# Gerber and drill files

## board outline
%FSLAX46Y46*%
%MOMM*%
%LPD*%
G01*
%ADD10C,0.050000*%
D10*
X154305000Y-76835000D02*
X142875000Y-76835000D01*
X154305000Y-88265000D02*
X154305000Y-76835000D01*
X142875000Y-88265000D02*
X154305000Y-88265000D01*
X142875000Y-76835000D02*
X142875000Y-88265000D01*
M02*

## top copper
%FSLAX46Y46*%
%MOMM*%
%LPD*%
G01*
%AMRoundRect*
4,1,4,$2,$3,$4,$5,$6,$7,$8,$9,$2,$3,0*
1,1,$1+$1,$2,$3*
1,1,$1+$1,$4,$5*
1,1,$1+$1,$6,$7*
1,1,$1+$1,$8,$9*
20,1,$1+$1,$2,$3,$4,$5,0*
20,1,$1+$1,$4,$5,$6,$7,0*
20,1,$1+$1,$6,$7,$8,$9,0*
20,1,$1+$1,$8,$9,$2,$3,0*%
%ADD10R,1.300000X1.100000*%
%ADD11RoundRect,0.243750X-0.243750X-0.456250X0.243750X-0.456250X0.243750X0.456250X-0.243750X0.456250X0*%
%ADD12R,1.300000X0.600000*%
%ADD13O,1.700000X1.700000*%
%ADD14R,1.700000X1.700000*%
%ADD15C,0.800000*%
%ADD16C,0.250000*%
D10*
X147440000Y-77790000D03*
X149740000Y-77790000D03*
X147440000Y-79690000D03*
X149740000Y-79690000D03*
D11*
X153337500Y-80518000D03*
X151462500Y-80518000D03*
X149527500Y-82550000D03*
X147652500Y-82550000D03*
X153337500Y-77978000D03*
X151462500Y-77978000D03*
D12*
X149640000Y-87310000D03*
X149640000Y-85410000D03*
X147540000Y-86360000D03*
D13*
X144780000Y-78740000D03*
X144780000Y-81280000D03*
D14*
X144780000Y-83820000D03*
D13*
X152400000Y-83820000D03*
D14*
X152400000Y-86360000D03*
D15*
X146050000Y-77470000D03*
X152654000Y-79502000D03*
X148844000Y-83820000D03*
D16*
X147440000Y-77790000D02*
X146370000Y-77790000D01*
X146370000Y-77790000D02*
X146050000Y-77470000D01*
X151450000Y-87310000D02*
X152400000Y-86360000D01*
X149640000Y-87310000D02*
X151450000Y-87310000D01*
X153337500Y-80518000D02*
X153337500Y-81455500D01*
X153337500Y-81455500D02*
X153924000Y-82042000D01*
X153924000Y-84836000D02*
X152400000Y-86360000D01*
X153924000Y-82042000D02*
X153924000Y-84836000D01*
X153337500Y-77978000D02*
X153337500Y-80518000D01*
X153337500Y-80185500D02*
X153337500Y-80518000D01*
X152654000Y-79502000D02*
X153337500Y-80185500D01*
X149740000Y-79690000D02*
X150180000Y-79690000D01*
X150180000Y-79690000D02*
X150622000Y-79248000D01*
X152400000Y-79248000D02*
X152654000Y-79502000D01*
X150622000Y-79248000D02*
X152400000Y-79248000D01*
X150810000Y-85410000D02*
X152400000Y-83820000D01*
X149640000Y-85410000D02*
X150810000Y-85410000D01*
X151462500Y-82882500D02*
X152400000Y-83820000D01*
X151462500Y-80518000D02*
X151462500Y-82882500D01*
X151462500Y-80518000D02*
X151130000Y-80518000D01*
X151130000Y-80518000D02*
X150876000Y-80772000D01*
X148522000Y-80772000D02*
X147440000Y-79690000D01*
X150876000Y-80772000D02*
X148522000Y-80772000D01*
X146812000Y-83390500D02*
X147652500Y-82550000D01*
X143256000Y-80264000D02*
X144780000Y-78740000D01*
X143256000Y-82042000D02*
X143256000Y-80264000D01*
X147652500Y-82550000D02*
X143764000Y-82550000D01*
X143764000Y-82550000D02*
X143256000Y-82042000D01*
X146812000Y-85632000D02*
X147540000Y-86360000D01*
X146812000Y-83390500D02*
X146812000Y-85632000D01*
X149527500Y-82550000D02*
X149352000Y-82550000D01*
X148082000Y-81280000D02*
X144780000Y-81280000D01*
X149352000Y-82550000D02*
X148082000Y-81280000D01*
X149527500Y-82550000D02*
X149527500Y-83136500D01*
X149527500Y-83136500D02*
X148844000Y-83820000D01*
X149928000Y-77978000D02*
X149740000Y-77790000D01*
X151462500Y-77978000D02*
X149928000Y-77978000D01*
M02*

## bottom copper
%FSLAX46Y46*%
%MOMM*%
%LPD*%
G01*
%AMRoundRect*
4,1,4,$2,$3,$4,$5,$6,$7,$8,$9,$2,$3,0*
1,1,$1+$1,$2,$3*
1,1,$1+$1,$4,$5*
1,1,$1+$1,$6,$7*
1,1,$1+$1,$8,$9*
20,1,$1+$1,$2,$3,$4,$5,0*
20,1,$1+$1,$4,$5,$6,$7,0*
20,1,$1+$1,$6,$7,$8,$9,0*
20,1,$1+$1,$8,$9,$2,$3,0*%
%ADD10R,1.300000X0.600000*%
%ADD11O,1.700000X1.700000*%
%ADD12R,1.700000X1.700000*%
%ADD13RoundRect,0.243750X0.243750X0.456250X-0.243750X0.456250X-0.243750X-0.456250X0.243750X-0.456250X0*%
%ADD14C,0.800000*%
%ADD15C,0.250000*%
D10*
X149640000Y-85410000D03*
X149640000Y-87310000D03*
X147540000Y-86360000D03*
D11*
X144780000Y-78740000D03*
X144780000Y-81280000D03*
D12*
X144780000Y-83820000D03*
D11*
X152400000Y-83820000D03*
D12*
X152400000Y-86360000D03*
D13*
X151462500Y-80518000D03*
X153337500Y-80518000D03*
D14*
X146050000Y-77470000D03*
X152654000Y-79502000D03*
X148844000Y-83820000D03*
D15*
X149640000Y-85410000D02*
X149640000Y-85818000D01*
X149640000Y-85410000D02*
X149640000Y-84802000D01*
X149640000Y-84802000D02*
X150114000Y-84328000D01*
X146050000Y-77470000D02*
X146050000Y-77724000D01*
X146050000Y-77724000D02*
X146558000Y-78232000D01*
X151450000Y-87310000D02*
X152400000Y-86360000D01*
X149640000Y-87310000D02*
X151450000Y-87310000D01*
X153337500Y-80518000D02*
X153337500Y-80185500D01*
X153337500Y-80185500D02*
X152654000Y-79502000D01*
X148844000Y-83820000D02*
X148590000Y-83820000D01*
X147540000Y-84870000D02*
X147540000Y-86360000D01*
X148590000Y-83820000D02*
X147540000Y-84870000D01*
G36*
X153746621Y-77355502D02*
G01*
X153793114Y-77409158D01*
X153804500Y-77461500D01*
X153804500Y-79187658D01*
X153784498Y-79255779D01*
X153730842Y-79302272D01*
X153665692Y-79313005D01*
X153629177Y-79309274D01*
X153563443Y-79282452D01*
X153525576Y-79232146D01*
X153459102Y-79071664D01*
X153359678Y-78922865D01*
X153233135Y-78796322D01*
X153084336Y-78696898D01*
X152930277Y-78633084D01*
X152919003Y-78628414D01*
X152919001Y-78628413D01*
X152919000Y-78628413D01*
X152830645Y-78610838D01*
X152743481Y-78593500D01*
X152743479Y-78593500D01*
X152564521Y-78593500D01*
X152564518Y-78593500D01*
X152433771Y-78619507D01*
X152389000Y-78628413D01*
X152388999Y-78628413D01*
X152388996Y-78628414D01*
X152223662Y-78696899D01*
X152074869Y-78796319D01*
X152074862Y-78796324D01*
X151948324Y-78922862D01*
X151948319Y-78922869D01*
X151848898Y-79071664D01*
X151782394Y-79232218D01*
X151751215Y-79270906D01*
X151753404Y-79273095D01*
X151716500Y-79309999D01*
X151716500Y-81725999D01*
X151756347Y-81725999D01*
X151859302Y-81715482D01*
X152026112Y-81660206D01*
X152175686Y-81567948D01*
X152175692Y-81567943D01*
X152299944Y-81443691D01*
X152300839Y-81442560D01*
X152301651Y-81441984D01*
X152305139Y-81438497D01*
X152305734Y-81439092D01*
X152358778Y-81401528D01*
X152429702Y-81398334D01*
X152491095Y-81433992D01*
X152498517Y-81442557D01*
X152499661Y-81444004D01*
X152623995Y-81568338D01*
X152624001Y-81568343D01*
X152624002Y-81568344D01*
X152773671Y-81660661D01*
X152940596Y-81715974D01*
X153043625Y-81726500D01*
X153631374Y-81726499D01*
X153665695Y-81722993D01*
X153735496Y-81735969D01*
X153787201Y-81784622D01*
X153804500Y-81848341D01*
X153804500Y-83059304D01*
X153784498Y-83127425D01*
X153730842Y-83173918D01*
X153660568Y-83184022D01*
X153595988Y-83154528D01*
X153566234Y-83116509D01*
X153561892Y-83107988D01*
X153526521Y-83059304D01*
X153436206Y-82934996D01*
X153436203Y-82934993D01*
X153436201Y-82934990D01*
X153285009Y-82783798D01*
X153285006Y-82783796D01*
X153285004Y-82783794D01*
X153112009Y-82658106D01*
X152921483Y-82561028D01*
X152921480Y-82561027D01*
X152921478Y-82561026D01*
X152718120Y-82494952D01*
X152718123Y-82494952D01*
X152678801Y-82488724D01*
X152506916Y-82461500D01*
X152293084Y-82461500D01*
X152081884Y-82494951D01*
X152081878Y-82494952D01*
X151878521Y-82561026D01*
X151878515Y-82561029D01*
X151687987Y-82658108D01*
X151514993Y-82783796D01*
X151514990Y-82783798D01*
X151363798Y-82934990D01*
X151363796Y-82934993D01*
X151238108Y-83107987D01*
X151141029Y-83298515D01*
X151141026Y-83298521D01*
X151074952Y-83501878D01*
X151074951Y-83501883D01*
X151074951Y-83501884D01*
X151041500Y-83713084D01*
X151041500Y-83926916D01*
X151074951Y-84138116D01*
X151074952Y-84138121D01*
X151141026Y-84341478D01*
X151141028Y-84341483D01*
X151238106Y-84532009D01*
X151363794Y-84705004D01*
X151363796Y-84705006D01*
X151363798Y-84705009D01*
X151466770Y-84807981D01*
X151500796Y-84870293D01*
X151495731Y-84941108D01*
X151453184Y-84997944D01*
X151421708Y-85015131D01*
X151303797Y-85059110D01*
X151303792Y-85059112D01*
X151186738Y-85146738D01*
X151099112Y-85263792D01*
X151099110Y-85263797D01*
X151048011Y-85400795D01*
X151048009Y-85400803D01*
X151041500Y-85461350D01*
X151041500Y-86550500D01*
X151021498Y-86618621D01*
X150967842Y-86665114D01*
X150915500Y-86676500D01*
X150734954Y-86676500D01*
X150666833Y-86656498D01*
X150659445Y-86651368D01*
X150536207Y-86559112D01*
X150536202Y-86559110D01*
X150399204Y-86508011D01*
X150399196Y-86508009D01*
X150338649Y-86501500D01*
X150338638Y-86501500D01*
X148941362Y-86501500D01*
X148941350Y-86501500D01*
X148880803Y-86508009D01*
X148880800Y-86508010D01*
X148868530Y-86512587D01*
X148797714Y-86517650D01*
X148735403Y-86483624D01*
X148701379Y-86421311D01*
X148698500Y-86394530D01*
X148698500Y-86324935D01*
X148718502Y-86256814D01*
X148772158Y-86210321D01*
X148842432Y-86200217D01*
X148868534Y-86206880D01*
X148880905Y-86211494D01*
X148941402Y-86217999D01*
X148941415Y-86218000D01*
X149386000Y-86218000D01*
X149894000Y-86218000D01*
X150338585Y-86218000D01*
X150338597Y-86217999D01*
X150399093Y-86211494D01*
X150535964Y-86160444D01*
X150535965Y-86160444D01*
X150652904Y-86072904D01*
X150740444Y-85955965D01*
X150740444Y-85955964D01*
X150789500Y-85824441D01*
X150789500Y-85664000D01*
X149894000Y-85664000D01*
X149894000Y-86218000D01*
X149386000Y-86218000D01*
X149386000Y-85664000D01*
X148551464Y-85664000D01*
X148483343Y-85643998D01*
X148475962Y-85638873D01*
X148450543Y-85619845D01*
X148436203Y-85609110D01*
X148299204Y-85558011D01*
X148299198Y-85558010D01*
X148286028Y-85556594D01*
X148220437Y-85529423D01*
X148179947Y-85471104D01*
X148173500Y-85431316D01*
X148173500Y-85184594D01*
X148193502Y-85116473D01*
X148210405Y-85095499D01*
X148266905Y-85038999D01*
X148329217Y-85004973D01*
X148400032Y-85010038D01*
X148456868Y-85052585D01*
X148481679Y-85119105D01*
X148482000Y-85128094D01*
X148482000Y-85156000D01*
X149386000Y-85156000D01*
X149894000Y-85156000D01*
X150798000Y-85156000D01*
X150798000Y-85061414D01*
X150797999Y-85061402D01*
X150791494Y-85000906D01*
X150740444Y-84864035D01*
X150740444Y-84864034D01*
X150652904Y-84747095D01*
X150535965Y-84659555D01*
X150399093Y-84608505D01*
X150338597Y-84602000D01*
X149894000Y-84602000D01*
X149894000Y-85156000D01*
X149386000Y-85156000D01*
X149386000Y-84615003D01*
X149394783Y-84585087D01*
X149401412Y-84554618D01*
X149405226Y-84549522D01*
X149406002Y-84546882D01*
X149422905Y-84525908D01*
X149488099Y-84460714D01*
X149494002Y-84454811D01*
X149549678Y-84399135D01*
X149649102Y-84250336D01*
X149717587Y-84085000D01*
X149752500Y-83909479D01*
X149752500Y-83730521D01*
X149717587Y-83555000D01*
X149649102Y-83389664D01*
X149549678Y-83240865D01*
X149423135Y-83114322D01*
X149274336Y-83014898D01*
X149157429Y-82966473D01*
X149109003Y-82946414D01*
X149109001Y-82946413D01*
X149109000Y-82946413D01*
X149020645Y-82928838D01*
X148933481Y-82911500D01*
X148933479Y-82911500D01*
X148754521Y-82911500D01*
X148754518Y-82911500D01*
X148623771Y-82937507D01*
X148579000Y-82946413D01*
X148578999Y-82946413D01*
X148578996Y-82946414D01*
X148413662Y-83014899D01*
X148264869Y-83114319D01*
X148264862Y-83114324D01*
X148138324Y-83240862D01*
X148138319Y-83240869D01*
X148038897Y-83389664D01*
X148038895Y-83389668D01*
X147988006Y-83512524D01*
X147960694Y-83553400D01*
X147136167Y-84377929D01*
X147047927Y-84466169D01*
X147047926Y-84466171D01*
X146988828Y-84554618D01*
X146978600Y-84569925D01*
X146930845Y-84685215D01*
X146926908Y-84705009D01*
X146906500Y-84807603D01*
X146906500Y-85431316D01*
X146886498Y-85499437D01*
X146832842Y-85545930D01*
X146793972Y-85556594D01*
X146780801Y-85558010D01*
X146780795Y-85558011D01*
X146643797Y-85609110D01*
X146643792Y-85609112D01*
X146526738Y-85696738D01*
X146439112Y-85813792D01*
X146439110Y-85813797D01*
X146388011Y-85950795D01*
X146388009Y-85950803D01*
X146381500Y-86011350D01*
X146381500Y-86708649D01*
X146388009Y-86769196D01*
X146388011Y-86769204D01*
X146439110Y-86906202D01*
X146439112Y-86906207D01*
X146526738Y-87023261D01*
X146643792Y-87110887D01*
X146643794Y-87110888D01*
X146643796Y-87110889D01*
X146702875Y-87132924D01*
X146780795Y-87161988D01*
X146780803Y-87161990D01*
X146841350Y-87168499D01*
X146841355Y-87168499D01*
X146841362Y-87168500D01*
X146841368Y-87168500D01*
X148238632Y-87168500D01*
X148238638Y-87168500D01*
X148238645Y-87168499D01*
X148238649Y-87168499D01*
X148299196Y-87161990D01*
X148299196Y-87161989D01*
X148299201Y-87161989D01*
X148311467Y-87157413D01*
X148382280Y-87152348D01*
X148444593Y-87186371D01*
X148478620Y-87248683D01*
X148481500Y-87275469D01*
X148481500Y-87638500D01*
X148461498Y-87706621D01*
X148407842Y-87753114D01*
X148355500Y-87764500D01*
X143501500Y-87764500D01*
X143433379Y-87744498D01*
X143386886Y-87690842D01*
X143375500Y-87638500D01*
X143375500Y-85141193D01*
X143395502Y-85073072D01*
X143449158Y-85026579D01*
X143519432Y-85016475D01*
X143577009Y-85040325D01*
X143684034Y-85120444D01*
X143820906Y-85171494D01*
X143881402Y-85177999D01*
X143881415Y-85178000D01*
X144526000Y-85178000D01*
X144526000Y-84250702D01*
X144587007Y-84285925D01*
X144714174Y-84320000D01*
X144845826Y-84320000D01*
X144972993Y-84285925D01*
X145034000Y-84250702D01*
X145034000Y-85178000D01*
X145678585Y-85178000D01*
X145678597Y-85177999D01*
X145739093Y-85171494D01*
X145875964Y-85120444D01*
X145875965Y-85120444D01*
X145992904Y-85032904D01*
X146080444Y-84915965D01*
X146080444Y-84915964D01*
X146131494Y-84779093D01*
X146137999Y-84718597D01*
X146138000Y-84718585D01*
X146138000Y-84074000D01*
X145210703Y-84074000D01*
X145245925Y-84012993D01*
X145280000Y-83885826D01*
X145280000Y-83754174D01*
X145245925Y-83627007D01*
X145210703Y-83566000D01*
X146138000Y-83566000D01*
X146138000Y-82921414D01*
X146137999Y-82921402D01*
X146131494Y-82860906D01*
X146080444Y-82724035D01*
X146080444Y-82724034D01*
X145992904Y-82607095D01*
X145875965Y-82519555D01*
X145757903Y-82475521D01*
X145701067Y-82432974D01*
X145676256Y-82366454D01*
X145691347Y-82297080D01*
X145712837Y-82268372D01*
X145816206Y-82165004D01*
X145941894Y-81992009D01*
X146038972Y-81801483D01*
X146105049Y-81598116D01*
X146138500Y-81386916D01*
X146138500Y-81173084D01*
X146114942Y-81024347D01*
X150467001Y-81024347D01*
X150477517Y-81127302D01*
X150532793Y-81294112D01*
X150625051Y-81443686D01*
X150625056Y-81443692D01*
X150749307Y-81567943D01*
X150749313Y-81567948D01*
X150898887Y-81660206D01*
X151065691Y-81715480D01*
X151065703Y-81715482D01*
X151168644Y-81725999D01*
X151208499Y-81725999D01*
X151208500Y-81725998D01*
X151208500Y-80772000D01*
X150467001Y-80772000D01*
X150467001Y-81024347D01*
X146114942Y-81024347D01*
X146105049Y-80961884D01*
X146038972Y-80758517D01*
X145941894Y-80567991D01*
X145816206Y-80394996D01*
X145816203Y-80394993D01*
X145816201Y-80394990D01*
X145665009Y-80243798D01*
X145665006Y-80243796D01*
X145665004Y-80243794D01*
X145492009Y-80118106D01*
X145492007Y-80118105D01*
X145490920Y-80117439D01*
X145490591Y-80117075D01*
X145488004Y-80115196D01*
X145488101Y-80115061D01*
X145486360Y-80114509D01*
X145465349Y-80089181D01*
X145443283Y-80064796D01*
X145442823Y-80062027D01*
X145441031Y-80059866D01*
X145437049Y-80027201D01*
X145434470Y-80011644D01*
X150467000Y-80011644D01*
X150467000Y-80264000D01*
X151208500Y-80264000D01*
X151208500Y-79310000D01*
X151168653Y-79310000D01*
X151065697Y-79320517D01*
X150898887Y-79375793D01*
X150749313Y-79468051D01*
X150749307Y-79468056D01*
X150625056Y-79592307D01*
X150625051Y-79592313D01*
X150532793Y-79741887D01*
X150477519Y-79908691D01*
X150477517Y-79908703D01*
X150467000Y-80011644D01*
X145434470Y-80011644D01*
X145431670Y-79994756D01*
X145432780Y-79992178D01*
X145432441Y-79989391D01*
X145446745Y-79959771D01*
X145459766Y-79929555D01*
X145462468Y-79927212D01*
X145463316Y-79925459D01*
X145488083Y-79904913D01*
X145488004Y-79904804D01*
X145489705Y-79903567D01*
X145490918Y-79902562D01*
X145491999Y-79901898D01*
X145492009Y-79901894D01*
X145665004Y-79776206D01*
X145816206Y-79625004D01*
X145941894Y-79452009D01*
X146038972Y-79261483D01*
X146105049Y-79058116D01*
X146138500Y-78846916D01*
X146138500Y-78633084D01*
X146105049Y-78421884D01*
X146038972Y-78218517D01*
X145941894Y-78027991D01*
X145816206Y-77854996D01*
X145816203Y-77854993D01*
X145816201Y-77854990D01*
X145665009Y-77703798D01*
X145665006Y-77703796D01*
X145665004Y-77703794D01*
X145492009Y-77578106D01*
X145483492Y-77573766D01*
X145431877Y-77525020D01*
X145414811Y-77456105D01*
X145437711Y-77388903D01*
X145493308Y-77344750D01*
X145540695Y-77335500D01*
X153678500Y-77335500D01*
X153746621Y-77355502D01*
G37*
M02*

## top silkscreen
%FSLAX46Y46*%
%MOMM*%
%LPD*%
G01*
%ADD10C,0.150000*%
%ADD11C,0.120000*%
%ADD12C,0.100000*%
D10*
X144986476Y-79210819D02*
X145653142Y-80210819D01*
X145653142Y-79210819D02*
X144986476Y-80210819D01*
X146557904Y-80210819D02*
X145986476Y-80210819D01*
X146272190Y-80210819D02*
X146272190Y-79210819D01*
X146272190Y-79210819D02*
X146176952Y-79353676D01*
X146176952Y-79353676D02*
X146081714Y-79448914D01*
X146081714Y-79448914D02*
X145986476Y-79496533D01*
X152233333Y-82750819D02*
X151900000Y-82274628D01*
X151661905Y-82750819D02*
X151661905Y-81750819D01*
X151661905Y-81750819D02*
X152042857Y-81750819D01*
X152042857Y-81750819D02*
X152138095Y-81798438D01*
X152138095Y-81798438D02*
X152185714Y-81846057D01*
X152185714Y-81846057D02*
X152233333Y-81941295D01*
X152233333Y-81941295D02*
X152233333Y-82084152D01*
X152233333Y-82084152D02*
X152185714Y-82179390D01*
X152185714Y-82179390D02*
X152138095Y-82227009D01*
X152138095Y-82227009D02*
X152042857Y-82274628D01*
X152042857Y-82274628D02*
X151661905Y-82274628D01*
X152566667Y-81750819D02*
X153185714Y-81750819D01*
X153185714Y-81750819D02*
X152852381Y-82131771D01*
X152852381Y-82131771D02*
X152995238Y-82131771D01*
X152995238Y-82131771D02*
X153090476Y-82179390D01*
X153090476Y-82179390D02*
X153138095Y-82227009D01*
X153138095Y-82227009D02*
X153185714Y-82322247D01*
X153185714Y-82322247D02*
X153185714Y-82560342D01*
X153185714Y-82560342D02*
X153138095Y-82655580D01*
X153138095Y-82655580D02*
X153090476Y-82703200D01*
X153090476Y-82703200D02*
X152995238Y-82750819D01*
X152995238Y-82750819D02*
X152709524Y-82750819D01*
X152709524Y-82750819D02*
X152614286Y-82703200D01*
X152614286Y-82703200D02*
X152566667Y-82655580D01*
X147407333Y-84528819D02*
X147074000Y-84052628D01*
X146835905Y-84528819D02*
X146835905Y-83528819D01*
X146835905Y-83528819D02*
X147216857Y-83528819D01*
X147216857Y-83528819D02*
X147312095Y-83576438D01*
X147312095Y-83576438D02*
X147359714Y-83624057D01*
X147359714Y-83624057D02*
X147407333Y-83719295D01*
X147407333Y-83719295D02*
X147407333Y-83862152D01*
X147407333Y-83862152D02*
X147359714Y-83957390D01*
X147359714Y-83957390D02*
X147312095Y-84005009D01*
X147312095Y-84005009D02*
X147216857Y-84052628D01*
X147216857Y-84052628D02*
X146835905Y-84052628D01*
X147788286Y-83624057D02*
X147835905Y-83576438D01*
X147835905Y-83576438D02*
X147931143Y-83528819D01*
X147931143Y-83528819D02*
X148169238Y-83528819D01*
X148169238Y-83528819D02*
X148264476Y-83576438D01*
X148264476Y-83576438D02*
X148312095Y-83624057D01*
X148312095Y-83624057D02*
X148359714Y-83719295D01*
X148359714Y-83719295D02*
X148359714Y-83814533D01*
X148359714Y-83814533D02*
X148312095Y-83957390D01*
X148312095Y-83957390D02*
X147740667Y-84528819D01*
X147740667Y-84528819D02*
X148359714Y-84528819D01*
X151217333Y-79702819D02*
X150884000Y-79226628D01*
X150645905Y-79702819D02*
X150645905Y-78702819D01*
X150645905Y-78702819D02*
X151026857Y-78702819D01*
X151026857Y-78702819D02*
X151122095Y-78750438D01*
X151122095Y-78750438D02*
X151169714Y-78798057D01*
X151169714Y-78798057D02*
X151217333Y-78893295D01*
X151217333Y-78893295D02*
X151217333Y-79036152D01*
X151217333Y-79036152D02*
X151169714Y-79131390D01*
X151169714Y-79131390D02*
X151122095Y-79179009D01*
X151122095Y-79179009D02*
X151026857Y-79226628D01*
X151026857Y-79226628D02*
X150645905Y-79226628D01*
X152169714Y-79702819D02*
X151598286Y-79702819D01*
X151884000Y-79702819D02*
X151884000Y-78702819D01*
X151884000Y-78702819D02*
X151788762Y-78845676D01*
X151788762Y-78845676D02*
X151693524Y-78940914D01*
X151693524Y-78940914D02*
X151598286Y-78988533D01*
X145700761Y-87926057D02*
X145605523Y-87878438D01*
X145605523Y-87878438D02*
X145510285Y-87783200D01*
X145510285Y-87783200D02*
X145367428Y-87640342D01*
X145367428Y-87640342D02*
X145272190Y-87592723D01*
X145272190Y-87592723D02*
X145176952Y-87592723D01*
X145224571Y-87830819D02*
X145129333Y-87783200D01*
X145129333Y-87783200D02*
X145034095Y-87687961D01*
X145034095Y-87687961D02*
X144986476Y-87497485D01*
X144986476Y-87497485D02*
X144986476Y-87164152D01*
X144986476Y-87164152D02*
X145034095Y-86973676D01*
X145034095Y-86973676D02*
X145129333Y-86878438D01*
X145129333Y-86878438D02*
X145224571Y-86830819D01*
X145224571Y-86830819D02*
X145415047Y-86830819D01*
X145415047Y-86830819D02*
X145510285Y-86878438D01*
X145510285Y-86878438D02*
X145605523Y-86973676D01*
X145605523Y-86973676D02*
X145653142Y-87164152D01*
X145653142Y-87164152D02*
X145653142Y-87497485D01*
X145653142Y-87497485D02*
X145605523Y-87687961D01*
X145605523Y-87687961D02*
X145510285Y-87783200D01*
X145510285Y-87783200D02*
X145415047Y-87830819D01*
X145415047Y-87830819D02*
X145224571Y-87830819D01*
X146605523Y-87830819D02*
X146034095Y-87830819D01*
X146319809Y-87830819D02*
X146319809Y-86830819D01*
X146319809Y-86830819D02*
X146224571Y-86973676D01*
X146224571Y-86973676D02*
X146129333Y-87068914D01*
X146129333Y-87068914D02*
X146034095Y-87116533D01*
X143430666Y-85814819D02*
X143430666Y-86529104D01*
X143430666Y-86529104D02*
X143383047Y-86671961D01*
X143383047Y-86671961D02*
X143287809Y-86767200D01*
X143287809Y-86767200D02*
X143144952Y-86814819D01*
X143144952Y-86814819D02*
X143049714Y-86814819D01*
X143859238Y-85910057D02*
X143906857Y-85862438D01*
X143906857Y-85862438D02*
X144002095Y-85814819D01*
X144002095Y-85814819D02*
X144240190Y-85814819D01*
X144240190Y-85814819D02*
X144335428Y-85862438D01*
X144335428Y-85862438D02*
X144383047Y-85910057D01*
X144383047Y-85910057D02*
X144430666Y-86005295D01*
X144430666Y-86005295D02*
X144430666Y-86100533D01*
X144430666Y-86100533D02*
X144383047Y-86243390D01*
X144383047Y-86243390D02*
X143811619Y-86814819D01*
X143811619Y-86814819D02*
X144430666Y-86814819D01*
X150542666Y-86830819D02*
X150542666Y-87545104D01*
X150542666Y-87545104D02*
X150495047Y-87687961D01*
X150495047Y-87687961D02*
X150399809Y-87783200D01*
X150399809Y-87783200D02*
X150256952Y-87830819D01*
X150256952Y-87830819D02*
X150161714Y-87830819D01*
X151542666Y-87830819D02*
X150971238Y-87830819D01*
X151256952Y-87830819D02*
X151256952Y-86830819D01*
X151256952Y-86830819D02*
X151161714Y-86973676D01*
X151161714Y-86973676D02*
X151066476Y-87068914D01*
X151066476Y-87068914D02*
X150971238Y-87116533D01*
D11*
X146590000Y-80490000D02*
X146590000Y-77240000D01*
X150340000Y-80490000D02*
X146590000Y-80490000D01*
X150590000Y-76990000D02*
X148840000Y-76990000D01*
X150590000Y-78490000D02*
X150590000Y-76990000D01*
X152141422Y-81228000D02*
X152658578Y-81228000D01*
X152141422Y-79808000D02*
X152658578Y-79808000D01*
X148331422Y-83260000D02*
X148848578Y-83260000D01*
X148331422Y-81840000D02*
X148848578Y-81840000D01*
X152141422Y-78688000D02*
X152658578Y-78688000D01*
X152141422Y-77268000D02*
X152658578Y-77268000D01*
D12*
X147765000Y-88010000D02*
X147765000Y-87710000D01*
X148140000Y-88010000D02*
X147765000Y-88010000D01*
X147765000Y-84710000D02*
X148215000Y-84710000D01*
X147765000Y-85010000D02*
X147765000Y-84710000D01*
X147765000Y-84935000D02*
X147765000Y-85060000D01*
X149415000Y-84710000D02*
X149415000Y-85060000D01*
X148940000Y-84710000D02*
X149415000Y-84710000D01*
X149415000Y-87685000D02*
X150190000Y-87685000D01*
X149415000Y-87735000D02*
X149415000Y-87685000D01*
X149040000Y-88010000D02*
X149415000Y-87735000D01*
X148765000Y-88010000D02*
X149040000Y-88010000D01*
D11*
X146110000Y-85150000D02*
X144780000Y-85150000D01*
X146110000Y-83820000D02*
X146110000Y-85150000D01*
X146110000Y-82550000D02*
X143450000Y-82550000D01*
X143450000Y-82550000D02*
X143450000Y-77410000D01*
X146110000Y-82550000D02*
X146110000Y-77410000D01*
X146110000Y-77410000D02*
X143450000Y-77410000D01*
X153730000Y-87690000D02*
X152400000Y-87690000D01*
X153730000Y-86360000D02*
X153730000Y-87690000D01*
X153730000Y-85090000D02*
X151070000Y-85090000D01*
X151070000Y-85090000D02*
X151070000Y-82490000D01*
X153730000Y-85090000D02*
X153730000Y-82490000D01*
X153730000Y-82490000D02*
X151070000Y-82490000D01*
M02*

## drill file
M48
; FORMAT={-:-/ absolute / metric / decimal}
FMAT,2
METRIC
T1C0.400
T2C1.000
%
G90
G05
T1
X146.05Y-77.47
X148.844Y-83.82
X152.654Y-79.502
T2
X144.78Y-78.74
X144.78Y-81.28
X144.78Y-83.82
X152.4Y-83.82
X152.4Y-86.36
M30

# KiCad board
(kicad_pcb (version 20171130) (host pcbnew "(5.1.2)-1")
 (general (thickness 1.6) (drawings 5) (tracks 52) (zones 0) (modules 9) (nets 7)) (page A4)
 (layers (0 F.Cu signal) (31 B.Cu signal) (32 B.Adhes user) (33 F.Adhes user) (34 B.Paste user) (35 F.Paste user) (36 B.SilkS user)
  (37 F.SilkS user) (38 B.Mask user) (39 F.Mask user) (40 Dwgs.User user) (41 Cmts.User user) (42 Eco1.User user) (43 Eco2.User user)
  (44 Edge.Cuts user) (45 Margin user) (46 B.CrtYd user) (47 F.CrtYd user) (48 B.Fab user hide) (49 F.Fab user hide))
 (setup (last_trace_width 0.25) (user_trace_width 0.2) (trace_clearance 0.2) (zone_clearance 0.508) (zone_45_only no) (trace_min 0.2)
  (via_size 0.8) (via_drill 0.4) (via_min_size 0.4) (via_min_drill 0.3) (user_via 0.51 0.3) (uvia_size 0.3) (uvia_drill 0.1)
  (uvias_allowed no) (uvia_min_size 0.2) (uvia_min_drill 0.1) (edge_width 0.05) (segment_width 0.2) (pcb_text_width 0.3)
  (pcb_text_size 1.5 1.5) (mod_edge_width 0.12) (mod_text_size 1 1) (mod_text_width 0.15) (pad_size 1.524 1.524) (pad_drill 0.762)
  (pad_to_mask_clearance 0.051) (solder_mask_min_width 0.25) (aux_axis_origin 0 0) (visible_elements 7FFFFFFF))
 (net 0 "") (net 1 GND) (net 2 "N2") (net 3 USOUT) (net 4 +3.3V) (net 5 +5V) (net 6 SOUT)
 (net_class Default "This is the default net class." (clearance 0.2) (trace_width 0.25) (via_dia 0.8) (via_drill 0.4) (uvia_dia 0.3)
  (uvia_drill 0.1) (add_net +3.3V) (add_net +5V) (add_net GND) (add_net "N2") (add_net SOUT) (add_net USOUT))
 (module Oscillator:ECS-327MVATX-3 (layer F.Cu) (at 148.59 78.74 180)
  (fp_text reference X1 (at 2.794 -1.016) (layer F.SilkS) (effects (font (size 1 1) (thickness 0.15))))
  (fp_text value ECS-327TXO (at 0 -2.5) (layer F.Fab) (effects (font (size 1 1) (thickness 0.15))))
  (fp_line (start 2 -1.75) (end 2 1.5) (layer F.SilkS) (width 0.12))
  (fp_line (start -1.75 -1.75) (end 2 -1.75) (layer F.SilkS) (width 0.12))
  (fp_line (start -2 1.75) (end -0.25 1.75) (layer F.SilkS) (width 0.12))
  (fp_line (start -2 0.25) (end -2 1.75) (layer F.SilkS) (width 0.12))
  (pad 2 smd rect (at 1.15 0.95 180) (size 1.3 1.1) (layers F.Cu F.Paste F.Mask) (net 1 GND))
  (pad 1 smd rect (at -1.15 0.95 180) (size 1.3 1.1) (layers F.Cu F.Paste F.Mask) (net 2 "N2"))
  (pad 3 smd rect (at 1.15 -0.95 180) (size 1.3 1.1) (layers F.Cu F.Paste F.Mask) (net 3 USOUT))
  (pad 4 smd rect (at -1.15 -0.95 180) (size 1.3 1.1) (layers F.Cu F.Paste F.Mask) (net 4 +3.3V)))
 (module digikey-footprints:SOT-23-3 (layer B.Cu) (at 148.59 86.36 180)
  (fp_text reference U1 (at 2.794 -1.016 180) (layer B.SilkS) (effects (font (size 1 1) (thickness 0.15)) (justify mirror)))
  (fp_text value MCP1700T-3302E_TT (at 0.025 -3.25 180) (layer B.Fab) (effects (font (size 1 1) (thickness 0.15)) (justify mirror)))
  (pad 1 smd rect (at -1.05 0.95 180) (size 1.3 0.6) (layers B.Cu B.Paste B.Mask) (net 1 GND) (solder_mask_margin 0.07))
  (pad 2 smd rect (at -1.05 -0.95 180) (size 1.3 0.6) (layers B.Cu B.Paste B.Mask) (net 4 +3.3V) (solder_mask_margin 0.07))
  (pad 3 smd rect (at 1.05 0 180) (size 1.3 0.6) (layers B.Cu B.Paste B.Mask) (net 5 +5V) (solder_mask_margin 0.07)))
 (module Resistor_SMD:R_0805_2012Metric (layer F.Cu) (at 152.4 80.518)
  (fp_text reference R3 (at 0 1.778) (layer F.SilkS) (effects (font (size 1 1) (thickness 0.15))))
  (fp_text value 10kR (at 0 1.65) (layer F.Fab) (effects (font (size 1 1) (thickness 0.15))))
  (fp_line (start -0.258578 0.71) (end 0.258578 0.71) (layer F.SilkS) (width 0.12))
  (fp_line (start -0.258578 -0.71) (end 0.258578 -0.71) (layer F.SilkS) (width 0.12))
  (pad 2 smd roundrect (at 0.9375 0) (size 0.975 1.4) (layers F.Cu F.Paste F.Mask) (roundrect_rratio 0.25) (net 4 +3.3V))
  (pad 1 smd roundrect (at -0.9375 0) (size 0.975 1.4) (layers F.Cu F.Paste F.Mask) (roundrect_rratio 0.25) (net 3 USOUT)))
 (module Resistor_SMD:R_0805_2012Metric (layer F.Cu) (at 148.59 82.55)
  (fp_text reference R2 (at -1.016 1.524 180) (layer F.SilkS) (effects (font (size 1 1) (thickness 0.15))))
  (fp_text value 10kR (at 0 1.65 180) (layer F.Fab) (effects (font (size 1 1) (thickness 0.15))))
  (fp_line (start -0.258578 0.71) (end 0.258578 0.71) (layer F.SilkS) (width 0.12))
  (fp_line (start -0.258578 -0.71) (end 0.258578 -0.71) (layer F.SilkS) (width 0.12))
  (pad 2 smd roundrect (at 0.9375 0) (size 0.975 1.4) (layers F.Cu F.Paste F.Mask) (roundrect_rratio 0.25) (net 5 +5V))
  (pad 1 smd roundrect (at -0.9375 0) (size 0.975 1.4) (layers F.Cu F.Paste F.Mask) (roundrect_rratio 0.25) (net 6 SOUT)))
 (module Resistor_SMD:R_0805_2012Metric (layer F.Cu) (at 152.4 77.978)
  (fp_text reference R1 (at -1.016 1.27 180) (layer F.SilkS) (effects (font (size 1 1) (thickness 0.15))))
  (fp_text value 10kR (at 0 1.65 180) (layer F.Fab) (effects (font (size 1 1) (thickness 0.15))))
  (fp_line (start -0.258578 0.71) (end 0.258578 0.71) (layer F.SilkS) (width 0.12))
  (fp_line (start -0.258578 -0.71) (end 0.258578 -0.71) (layer F.SilkS) (width 0.12))
  (pad 2 smd roundrect (at 0.9375 0) (size 0.975 1.4) (layers F.Cu F.Paste F.Mask) (roundrect_rratio 0.25) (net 4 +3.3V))
  (pad 1 smd roundrect (at -0.9375 0) (size 0.975 1.4) (layers F.Cu F.Paste F.Mask) (roundrect_rratio 0.25) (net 2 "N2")))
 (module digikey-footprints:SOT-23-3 (layer F.Cu) (at 148.59 86.36 180)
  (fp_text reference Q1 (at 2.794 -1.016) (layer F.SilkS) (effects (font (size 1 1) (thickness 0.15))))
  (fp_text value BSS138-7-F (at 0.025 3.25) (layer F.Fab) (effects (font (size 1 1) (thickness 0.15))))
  (fp_line (start 0.825 -1.65) (end 0.825 -1.35) (layer F.SilkS) (width 0.1))
  (fp_line (start 0.45 -1.65) (end 0.825 -1.65) (layer F.SilkS) (width 0.1))
  (fp_line (start 0.825 1.65) (end 0.375 1.65) (layer F.SilkS) (width 0.1))
  (fp_line (start 0.825 1.35) (end 0.825 1.65) (layer F.SilkS) (width 0.1))
  (fp_line (start 0.825 1.425) (end 0.825 1.3) (layer F.SilkS) (width 0.1))
  (fp_line (start -0.825 1.65) (end -0.825 1.3) (layer F.SilkS) (width 0.1))
  (fp_line (start -0.35 1.65) (end -0.825 1.65) (layer F.SilkS) (width 0.1))
  (fp_line (start -0.825 -1.325) (end -1.6 -1.325) (layer F.SilkS) (width 0.1))
  (fp_line (start -0.825 -1.375) (end -0.825 -1.325) (layer F.SilkS) (width 0.1))
  (fp_line (start -0.45 -1.65) (end -0.825 -1.375) (layer F.SilkS) (width 0.1))
  (fp_line (start -0.175 -1.65) (end -0.45 -1.65) (layer F.SilkS) (width 0.1))
  (pad 1 smd rect (at -1.05 -0.95 180) (size 1.3 0.6) (layers F.Cu F.Paste F.Mask) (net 4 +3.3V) (solder_mask_margin 0.07))
  (pad 2 smd rect (at -1.05 0.95 180) (size 1.3 0.6) (layers F.Cu F.Paste F.Mask) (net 3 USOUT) (solder_mask_margin 0.07))
  (pad 3 smd rect (at 1.05 0 180) (size 1.3 0.6) (layers F.Cu F.Paste F.Mask) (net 6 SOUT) (solder_mask_margin 0.07)))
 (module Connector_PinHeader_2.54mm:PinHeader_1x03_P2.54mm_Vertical (layer F.Cu) (at 144.78 83.82 180)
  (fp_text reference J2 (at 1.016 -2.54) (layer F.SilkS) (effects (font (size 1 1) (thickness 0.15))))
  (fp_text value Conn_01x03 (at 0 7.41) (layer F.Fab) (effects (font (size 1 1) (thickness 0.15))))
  (fp_line (start -1.33 -1.33) (end 0 -1.33) (layer F.SilkS) (width 0.12))
  (fp_line (start -1.33 0) (end -1.33 -1.33) (layer F.SilkS) (width 0.12))
  (fp_line (start -1.33 1.27) (end 1.33 1.27) (layer F.SilkS) (width 0.12))
  (fp_line (start 1.33 1.27) (end 1.33 6.41) (layer F.SilkS) (width 0.12))
  (fp_line (start -1.33 1.27) (end -1.33 6.41) (layer F.SilkS) (width 0.12))
  (fp_line (start -1.33 6.41) (end 1.33 6.41) (layer F.SilkS) (width 0.12))
  (pad 3 thru_hole oval (at 0 5.08 180) (size 1.7 1.7) (drill 1) (layers *.Cu *.Mask) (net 6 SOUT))
  (pad 2 thru_hole oval (at 0 2.54 180) (size 1.7 1.7) (drill 1) (layers *.Cu *.Mask) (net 5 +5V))
  (pad 1 thru_hole rect (at 0 0 180) (size 1.7 1.7) (drill 1) (layers *.Cu *.Mask) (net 1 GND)))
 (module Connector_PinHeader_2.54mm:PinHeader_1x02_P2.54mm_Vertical (layer F.Cu) (at 152.4 86.36 180)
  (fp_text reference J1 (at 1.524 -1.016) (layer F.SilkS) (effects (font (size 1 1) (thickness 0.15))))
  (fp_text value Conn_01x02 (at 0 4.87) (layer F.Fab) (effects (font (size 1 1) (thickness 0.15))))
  (fp_line (start -1.33 -1.33) (end 0 -1.33) (layer F.SilkS) (width 0.12))
  (fp_line (start -1.33 0) (end -1.33 -1.33) (layer F.SilkS) (width 0.12))
  (fp_line (start -1.33 1.27) (end 1.33 1.27) (layer F.SilkS) (width 0.12))
  (fp_line (start 1.33 1.27) (end 1.33 3.87) (layer F.SilkS) (width 0.12))
  (fp_line (start -1.33 1.27) (end -1.33 3.87) (layer F.SilkS) (width 0.12))
  (fp_line (start -1.33 3.87) (end 1.33 3.87) (layer F.SilkS) (width 0.12))
  (pad 2 thru_hole oval (at 0 2.54 180) (size 1.7 1.7) (drill 1) (layers *.Cu *.Mask) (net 3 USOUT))
  (pad 1 thru_hole rect (at 0 0 180) (size 1.7 1.7) (drill 1) (layers *.Cu *.Mask) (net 4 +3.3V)))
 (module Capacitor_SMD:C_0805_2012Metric (layer B.Cu) (at 152.4 80.518 180)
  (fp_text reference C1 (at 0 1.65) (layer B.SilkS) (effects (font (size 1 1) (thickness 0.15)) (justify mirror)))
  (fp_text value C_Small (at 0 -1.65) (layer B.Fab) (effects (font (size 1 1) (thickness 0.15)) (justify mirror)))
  (pad 2 smd roundrect (at 0.9375 0 180) (size 0.975 1.4) (layers B.Cu B.Paste B.Mask) (roundrect_rratio 0.25) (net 1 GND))
  (pad 1 smd roundrect (at -0.9375 0 180) (size 0.975 1.4) (layers B.Cu B.Paste B.Mask) (roundrect_rratio 0.25) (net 4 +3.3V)))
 (gr_line (start 154.305 76.835) (end 142.875 76.835) (layer Edge.Cuts) (width 0.05))
 (gr_line (start 154.305 88.265) (end 154.305 76.835) (layer Edge.Cuts) (width 0.05))
 (gr_line (start 142.875 88.265) (end 154.305 88.265) (layer Edge.Cuts) (width 0.05))
 (gr_line (start 142.875 76.835) (end 142.875 88.265) (layer Edge.Cuts) (width 0.05))
 (segment (start 149.64 85.41) (end 149.64 85.818) (width 0.25) (layer B.Cu) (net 1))
 (via (at 146.05 77.47) (size 0.8) (drill 0.4) (layers F.Cu B.Cu) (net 1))
 (segment (start 147.44 77.79) (end 146.37 77.79) (width 0.25) (layer F.Cu) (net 1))
 (segment (start 146.37 77.79) (end 146.05 77.47) (width 0.25) (layer F.Cu) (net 1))
 (segment (start 149.64 85.41) (end 149.64 84.802) (width 0.25) (layer B.Cu) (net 1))
 (segment (start 149.64 84.802) (end 150.114 84.328) (width 0.25) (layer B.Cu) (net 1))
 (segment (start 146.05 77.47) (end 146.05 77.724) (width 0.25) (layer B.Cu) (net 1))
 (segment (start 146.05 77.724) (end 146.558 78.232) (width 0.25) (layer B.Cu) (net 1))
 (segment (start 151.45 87.31) (end 152.4 86.36) (width 0.25) (layer F.Cu) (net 4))
 (segment (start 149.64 87.31) (end 151.45 87.31) (width 0.25) (layer F.Cu) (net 4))
 (segment (start 151.45 87.31) (end 152.4 86.36) (width 0.25) (layer B.Cu) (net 4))
 (segment (start 149.64 87.31) (end 151.45 87.31) (width 0.25) (layer B.Cu) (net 4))
 (segment (start 153.3375 80.518) (end 153.3375 81.4555) (width 0.25) (layer F.Cu) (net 4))
 (segment (start 153.3375 81.4555) (end 153.924 82.042) (width 0.25) (layer F.Cu) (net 4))
 (segment (start 153.924 84.836) (end 152.4 86.36) (width 0.25) (layer F.Cu) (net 4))
 (segment (start 153.924 82.042) (end 153.924 84.836) (width 0.25) (layer F.Cu) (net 4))
 (segment (start 153.3375 77.978) (end 153.3375 80.518) (width 0.25) (layer F.Cu) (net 4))
 (via (at 152.654 79.502) (size 0.8) (drill 0.4) (layers F.Cu B.Cu) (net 4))
 (segment (start 153.3375 80.518) (end 153.3375 80.1855) (width 0.25) (layer B.Cu) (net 4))
 (segment (start 153.3375 80.1855) (end 152.654 79.502) (width 0.25) (layer B.Cu) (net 4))
 (segment (start 153.3375 80.1855) (end 153.3375 80.518) (width 0.25) (layer F.Cu) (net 4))
 (segment (start 152.654 79.502) (end 153.3375 80.1855) (width 0.25) (layer F.Cu) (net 4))
 (segment (start 149.74 79.69) (end 150.18 79.69) (width 0.25) (layer F.Cu) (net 4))
 (segment (start 150.18 79.69) (end 150.622 79.248) (width 0.25) (layer F.Cu) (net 4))
 (segment (start 152.4 79.248) (end 152.654 79.502) (width 0.25) (layer F.Cu) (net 4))
 (segment (start 150.622 79.248) (end 152.4 79.248) (width 0.25) (layer F.Cu) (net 4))
 (segment (start 150.81 85.41) (end 152.4 83.82) (width 0.25) (layer F.Cu) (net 3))
 (segment (start 149.64 85.41) (end 150.81 85.41) (width 0.25) (layer F.Cu) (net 3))
 (segment (start 151.4625 82.8825) (end 152.4 83.82) (width 0.25) (layer F.Cu) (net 3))
 (segment (start 151.4625 80.518) (end 151.4625 82.8825) (width 0.25) (layer F.Cu) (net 3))
 (segment (start 151.4625 80.518) (end 151.13 80.518) (width 0.25) (layer F.Cu) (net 3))
 (segment (start 151.13 80.518) (end 150.876 80.772) (width 0.25) (layer F.Cu) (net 3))
 (segment (start 148.522 80.772) (end 147.44 79.69) (width 0.25) (layer F.Cu) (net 3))
 (segment (start 150.876 80.772) (end 148.522 80.772) (width 0.25) (layer F.Cu) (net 3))
 (segment (start 146.812 83.3905) (end 147.6525 82.55) (width 0.25) (layer F.Cu) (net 6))
 (segment (start 143.256 80.264) (end 144.78 78.74) (width 0.25) (layer F.Cu) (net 6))
 (segment (start 143.256 82.042) (end 143.256 80.264) (width 0.25) (layer F.Cu) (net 6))
 (segment (start 147.6525 82.55) (end 143.764 82.55) (width 0.25) (layer F.Cu) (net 6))
 (segment (start 143.764 82.55) (end 143.256 82.042) (width 0.25) (layer F.Cu) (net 6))
 (segment (start 146.812 85.632) (end 147.54 86.36) (width 0.25) (layer F.Cu) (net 6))
 (segment (start 146.812 83.3905) (end 146.812 85.632) (width 0.25) (layer F.Cu) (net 6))
 (segment (start 149.5275 82.55) (end 149.352 82.55) (width 0.25) (layer F.Cu) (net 5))
 (segment (start 148.082 81.28) (end 144.78 81.28) (width 0.25) (layer F.Cu) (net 5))
 (segment (start 149.352 82.55) (end 148.082 81.28) (width 0.25) (layer F.Cu) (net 5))
 (via (at 148.844 83.82) (size 0.8) (drill 0.4) (layers F.Cu B.Cu) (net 5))
 (segment (start 149.5275 82.55) (end 149.5275 83.1365) (width 0.25) (layer F.Cu) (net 5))
 (segment (start 149.5275 83.1365) (end 148.844 83.82) (width 0.25) (layer F.Cu) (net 5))
 (segment (start 148.844 83.82) (end 148.59 83.82) (width 0.25) (layer B.Cu) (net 5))
 (segment (start 147.54 84.87) (end 147.54 86.36) (width 0.25) (layer B.Cu) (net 5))
 (segment (start 148.59 83.82) (end 147.54 84.87) (width 0.25) (layer B.Cu) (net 5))
 (segment (start 149.928 77.978) (end 149.74 77.79) (width 0.25) (layer F.Cu) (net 2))
 (segment (start 151.4625 77.978) (end 149.928 77.978) (width 0.25) (layer F.Cu) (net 2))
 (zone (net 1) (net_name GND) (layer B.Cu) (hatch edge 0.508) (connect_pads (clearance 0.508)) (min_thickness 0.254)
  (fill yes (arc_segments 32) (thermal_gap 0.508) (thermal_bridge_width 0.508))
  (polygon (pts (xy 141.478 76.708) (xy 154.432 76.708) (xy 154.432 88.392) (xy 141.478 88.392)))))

